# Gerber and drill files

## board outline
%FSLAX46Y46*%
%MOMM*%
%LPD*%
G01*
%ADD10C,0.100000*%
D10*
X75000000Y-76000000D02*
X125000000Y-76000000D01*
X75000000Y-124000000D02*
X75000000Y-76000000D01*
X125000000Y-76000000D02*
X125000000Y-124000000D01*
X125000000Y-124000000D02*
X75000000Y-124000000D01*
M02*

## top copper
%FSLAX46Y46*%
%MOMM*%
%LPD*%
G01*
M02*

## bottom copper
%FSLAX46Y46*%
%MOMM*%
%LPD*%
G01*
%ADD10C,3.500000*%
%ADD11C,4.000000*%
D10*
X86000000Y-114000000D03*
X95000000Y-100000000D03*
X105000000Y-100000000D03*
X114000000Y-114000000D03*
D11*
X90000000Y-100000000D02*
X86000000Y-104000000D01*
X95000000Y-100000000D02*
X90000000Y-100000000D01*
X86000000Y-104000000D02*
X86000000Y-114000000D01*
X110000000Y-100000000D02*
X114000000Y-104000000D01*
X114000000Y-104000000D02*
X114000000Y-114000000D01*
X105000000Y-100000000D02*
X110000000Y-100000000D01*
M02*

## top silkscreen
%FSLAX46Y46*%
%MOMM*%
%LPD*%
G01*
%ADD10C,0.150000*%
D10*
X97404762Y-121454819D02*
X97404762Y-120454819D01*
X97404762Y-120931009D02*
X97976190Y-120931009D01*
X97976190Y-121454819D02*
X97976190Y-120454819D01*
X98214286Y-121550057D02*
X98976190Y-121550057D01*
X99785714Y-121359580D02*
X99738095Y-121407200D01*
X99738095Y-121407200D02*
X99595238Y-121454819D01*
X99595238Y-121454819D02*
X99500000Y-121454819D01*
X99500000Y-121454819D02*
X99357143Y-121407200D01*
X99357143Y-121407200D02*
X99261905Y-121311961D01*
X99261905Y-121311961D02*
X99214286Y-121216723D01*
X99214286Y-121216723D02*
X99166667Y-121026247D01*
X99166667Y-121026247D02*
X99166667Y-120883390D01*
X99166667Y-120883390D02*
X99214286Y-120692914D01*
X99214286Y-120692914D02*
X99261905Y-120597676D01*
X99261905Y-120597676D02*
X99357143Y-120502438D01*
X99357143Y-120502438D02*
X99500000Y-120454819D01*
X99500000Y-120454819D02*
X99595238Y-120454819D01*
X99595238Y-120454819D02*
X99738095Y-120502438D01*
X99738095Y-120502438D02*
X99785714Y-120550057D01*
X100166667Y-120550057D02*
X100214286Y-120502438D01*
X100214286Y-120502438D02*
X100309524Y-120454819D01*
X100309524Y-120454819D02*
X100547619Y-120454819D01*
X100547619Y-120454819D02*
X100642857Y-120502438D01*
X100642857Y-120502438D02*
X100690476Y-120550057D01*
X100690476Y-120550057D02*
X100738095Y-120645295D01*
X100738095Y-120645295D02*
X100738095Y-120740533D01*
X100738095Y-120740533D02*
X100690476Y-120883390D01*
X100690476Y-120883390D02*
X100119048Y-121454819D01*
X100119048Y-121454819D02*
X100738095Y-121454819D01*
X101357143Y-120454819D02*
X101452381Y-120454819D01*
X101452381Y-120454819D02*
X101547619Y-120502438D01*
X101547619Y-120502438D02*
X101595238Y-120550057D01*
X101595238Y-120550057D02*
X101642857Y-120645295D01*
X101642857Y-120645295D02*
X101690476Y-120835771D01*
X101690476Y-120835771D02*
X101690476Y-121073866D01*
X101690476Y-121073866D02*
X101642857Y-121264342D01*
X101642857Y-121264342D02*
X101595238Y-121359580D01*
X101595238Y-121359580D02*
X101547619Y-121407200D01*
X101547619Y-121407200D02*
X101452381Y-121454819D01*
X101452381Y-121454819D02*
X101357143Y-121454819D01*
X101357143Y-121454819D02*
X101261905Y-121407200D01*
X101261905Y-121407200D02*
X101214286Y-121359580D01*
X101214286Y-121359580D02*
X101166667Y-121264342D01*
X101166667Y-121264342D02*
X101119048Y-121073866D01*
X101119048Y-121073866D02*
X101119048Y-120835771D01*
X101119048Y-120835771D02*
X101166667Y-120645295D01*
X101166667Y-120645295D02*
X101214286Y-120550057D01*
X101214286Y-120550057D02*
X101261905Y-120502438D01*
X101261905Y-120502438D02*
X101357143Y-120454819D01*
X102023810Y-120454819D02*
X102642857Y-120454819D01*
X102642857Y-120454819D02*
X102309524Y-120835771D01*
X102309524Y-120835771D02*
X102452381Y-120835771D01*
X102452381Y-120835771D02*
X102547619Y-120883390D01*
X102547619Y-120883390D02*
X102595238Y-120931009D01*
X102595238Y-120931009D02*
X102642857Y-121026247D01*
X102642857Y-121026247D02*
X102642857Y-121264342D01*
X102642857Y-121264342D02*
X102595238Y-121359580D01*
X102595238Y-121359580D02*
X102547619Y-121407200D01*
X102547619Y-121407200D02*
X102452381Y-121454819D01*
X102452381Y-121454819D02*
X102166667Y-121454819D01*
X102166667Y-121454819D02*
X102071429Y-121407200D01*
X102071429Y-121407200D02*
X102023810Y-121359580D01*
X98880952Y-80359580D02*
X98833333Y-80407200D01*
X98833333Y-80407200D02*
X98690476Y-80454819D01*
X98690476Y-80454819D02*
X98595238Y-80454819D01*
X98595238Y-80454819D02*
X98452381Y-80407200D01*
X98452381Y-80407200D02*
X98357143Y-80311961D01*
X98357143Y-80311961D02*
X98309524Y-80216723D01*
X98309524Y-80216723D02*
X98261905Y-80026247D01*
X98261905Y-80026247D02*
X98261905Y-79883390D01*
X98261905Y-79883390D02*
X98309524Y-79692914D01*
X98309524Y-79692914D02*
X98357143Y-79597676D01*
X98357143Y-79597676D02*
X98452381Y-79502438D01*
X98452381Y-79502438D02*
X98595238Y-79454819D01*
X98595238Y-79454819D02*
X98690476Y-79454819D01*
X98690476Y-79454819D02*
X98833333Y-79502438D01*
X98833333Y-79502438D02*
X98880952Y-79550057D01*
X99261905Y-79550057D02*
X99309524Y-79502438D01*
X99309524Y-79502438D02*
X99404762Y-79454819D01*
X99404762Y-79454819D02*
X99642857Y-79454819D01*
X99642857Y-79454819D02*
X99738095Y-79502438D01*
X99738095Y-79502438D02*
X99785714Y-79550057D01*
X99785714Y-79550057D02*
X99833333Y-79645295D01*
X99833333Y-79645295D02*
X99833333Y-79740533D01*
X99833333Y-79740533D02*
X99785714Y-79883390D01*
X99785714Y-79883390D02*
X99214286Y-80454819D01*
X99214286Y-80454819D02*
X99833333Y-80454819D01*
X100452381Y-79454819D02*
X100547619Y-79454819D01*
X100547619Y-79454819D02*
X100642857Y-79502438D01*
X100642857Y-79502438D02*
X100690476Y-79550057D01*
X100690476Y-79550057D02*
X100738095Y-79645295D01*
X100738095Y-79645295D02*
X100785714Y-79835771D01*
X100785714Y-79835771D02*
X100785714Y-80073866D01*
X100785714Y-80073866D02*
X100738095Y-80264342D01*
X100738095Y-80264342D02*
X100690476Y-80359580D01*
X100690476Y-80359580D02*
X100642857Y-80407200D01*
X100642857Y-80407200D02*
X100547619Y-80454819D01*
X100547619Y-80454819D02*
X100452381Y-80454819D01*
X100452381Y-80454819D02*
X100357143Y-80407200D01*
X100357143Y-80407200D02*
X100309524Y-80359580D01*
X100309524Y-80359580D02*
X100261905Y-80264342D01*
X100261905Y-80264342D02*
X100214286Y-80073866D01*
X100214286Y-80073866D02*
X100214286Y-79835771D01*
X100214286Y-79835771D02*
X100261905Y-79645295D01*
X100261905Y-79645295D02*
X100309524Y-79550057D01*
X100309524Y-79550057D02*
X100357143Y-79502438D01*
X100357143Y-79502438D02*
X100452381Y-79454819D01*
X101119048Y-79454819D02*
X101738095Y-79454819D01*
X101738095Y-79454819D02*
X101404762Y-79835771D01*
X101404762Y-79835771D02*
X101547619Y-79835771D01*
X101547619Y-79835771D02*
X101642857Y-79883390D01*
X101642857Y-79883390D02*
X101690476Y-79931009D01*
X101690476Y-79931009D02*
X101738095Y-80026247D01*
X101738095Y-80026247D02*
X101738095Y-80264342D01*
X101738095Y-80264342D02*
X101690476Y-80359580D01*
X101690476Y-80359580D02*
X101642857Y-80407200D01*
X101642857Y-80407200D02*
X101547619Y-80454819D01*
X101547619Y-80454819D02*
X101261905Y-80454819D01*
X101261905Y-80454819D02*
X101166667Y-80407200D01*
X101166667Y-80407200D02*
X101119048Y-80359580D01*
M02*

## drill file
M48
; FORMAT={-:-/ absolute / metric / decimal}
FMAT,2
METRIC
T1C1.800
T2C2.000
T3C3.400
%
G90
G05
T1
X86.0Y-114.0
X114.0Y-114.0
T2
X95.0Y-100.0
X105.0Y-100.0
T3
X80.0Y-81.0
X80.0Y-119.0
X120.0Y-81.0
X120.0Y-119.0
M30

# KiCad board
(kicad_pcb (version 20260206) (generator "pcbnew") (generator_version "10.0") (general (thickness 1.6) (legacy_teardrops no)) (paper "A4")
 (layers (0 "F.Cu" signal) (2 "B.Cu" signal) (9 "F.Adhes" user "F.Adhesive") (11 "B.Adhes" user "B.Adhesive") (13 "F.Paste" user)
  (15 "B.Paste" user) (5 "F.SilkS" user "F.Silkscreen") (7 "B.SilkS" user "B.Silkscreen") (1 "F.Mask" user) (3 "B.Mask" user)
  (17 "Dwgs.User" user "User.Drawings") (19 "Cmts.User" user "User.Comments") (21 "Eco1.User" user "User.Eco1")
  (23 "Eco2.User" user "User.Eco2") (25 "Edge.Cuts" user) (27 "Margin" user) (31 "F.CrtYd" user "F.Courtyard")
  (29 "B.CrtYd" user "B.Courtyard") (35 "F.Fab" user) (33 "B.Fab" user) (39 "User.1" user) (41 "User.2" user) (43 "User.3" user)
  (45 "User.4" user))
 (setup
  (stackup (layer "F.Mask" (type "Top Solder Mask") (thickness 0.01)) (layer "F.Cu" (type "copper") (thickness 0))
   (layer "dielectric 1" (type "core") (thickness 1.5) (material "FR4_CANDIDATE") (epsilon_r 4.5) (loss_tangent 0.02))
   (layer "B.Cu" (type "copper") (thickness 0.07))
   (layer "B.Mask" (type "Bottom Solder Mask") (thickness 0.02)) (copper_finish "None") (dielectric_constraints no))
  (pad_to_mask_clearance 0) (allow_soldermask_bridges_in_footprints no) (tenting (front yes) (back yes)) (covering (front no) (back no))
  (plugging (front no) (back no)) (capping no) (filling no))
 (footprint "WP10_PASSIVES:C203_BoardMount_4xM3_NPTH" (layer "F.Cu") (at 100 100)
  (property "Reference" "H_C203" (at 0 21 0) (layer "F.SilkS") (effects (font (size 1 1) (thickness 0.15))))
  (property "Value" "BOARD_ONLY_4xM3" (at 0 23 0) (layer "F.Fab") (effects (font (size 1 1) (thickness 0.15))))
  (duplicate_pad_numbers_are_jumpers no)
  (pad "" np_thru_hole circle (at -20 -19) (size 3.4 3.4) (drill 3.4) (layers "*.Cu" "*.Mask"))
  (pad "" np_thru_hole circle (at -20 19) (size 3.4 3.4) (drill 3.4) (layers "*.Cu" "*.Mask"))
  (pad "" np_thru_hole circle (at 20 -19) (size 3.4 3.4) (drill 3.4) (layers "*.Cu" "*.Mask"))
  (pad "" np_thru_hole circle (at 20 19) (size 3.4 3.4) (drill 3.4) (layers "*.Cu" "*.Mask")))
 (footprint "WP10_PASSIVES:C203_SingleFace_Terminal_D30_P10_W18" (layer "F.Cu") (at 100 100)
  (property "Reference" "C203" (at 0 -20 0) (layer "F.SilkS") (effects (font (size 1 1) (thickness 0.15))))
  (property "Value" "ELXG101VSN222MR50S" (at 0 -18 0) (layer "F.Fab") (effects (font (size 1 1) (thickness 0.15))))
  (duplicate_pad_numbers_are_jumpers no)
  (pad "" np_thru_hole circle (at -14 14) (size 1.8 1.8) (drill 1.8) (layers "*.Cu" "F.Mask"))
  (pad "" np_thru_hole circle (at -5 0) (size 2 2) (drill 2) (layers "*.Cu" "F.Mask"))
  (pad "" np_thru_hole circle (at 5 0) (size 2 2) (drill 2) (layers "*.Cu" "F.Mask"))
  (pad "" np_thru_hole circle (at 14 14) (size 1.8 1.8) (drill 1.8) (layers "*.Cu" "F.Mask"))
  (pad "1" smd circle (at -14 14) (size 3.5 3.5) (layers "B.Cu" "B.Mask") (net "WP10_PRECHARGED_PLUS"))
  (pad "1" smd circle (at -5 0) (size 3.5 3.5) (layers "B.Cu" "B.Mask") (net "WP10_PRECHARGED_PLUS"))
  (pad "2" smd circle (at 5 0) (size 3.5 3.5) (layers "B.Cu" "B.Mask") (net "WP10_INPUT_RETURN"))
  (pad "2" smd circle (at 14 14) (size 3.5 3.5) (layers "B.Cu" "B.Mask") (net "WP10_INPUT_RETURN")))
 (gr_line (start 75 76) (end 125 76) (stroke (width 0.1) (type default)) (layer "Edge.Cuts"))
 (gr_line (start 75 124) (end 75 76) (stroke (width 0.1) (type default)) (layer "Edge.Cuts"))
 (gr_line (start 125 76) (end 125 124) (stroke (width 0.1) (type default)) (layer "Edge.Cuts"))
 (gr_line (start 125 124) (end 75 124) (stroke (width 0.1) (type default)) (layer "Edge.Cuts"))
 (segment (start 90 100) (end 86 104) (width 4) (layer "B.Cu") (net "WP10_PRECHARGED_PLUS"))
 (segment (start 95 100) (end 90 100) (width 4) (layer "B.Cu") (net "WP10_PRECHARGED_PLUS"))
 (segment (start 86 104) (end 86 114) (width 4) (layer "B.Cu") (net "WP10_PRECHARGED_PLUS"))
 (segment (start 110 100) (end 114 104) (width 4) (layer "B.Cu") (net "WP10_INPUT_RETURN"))
 (segment (start 114 104) (end 114 114) (width 4) (layer "B.Cu") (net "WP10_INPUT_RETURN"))
 (segment (start 105 100) (end 110 100) (width 4) (layer "B.Cu") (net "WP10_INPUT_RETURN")))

